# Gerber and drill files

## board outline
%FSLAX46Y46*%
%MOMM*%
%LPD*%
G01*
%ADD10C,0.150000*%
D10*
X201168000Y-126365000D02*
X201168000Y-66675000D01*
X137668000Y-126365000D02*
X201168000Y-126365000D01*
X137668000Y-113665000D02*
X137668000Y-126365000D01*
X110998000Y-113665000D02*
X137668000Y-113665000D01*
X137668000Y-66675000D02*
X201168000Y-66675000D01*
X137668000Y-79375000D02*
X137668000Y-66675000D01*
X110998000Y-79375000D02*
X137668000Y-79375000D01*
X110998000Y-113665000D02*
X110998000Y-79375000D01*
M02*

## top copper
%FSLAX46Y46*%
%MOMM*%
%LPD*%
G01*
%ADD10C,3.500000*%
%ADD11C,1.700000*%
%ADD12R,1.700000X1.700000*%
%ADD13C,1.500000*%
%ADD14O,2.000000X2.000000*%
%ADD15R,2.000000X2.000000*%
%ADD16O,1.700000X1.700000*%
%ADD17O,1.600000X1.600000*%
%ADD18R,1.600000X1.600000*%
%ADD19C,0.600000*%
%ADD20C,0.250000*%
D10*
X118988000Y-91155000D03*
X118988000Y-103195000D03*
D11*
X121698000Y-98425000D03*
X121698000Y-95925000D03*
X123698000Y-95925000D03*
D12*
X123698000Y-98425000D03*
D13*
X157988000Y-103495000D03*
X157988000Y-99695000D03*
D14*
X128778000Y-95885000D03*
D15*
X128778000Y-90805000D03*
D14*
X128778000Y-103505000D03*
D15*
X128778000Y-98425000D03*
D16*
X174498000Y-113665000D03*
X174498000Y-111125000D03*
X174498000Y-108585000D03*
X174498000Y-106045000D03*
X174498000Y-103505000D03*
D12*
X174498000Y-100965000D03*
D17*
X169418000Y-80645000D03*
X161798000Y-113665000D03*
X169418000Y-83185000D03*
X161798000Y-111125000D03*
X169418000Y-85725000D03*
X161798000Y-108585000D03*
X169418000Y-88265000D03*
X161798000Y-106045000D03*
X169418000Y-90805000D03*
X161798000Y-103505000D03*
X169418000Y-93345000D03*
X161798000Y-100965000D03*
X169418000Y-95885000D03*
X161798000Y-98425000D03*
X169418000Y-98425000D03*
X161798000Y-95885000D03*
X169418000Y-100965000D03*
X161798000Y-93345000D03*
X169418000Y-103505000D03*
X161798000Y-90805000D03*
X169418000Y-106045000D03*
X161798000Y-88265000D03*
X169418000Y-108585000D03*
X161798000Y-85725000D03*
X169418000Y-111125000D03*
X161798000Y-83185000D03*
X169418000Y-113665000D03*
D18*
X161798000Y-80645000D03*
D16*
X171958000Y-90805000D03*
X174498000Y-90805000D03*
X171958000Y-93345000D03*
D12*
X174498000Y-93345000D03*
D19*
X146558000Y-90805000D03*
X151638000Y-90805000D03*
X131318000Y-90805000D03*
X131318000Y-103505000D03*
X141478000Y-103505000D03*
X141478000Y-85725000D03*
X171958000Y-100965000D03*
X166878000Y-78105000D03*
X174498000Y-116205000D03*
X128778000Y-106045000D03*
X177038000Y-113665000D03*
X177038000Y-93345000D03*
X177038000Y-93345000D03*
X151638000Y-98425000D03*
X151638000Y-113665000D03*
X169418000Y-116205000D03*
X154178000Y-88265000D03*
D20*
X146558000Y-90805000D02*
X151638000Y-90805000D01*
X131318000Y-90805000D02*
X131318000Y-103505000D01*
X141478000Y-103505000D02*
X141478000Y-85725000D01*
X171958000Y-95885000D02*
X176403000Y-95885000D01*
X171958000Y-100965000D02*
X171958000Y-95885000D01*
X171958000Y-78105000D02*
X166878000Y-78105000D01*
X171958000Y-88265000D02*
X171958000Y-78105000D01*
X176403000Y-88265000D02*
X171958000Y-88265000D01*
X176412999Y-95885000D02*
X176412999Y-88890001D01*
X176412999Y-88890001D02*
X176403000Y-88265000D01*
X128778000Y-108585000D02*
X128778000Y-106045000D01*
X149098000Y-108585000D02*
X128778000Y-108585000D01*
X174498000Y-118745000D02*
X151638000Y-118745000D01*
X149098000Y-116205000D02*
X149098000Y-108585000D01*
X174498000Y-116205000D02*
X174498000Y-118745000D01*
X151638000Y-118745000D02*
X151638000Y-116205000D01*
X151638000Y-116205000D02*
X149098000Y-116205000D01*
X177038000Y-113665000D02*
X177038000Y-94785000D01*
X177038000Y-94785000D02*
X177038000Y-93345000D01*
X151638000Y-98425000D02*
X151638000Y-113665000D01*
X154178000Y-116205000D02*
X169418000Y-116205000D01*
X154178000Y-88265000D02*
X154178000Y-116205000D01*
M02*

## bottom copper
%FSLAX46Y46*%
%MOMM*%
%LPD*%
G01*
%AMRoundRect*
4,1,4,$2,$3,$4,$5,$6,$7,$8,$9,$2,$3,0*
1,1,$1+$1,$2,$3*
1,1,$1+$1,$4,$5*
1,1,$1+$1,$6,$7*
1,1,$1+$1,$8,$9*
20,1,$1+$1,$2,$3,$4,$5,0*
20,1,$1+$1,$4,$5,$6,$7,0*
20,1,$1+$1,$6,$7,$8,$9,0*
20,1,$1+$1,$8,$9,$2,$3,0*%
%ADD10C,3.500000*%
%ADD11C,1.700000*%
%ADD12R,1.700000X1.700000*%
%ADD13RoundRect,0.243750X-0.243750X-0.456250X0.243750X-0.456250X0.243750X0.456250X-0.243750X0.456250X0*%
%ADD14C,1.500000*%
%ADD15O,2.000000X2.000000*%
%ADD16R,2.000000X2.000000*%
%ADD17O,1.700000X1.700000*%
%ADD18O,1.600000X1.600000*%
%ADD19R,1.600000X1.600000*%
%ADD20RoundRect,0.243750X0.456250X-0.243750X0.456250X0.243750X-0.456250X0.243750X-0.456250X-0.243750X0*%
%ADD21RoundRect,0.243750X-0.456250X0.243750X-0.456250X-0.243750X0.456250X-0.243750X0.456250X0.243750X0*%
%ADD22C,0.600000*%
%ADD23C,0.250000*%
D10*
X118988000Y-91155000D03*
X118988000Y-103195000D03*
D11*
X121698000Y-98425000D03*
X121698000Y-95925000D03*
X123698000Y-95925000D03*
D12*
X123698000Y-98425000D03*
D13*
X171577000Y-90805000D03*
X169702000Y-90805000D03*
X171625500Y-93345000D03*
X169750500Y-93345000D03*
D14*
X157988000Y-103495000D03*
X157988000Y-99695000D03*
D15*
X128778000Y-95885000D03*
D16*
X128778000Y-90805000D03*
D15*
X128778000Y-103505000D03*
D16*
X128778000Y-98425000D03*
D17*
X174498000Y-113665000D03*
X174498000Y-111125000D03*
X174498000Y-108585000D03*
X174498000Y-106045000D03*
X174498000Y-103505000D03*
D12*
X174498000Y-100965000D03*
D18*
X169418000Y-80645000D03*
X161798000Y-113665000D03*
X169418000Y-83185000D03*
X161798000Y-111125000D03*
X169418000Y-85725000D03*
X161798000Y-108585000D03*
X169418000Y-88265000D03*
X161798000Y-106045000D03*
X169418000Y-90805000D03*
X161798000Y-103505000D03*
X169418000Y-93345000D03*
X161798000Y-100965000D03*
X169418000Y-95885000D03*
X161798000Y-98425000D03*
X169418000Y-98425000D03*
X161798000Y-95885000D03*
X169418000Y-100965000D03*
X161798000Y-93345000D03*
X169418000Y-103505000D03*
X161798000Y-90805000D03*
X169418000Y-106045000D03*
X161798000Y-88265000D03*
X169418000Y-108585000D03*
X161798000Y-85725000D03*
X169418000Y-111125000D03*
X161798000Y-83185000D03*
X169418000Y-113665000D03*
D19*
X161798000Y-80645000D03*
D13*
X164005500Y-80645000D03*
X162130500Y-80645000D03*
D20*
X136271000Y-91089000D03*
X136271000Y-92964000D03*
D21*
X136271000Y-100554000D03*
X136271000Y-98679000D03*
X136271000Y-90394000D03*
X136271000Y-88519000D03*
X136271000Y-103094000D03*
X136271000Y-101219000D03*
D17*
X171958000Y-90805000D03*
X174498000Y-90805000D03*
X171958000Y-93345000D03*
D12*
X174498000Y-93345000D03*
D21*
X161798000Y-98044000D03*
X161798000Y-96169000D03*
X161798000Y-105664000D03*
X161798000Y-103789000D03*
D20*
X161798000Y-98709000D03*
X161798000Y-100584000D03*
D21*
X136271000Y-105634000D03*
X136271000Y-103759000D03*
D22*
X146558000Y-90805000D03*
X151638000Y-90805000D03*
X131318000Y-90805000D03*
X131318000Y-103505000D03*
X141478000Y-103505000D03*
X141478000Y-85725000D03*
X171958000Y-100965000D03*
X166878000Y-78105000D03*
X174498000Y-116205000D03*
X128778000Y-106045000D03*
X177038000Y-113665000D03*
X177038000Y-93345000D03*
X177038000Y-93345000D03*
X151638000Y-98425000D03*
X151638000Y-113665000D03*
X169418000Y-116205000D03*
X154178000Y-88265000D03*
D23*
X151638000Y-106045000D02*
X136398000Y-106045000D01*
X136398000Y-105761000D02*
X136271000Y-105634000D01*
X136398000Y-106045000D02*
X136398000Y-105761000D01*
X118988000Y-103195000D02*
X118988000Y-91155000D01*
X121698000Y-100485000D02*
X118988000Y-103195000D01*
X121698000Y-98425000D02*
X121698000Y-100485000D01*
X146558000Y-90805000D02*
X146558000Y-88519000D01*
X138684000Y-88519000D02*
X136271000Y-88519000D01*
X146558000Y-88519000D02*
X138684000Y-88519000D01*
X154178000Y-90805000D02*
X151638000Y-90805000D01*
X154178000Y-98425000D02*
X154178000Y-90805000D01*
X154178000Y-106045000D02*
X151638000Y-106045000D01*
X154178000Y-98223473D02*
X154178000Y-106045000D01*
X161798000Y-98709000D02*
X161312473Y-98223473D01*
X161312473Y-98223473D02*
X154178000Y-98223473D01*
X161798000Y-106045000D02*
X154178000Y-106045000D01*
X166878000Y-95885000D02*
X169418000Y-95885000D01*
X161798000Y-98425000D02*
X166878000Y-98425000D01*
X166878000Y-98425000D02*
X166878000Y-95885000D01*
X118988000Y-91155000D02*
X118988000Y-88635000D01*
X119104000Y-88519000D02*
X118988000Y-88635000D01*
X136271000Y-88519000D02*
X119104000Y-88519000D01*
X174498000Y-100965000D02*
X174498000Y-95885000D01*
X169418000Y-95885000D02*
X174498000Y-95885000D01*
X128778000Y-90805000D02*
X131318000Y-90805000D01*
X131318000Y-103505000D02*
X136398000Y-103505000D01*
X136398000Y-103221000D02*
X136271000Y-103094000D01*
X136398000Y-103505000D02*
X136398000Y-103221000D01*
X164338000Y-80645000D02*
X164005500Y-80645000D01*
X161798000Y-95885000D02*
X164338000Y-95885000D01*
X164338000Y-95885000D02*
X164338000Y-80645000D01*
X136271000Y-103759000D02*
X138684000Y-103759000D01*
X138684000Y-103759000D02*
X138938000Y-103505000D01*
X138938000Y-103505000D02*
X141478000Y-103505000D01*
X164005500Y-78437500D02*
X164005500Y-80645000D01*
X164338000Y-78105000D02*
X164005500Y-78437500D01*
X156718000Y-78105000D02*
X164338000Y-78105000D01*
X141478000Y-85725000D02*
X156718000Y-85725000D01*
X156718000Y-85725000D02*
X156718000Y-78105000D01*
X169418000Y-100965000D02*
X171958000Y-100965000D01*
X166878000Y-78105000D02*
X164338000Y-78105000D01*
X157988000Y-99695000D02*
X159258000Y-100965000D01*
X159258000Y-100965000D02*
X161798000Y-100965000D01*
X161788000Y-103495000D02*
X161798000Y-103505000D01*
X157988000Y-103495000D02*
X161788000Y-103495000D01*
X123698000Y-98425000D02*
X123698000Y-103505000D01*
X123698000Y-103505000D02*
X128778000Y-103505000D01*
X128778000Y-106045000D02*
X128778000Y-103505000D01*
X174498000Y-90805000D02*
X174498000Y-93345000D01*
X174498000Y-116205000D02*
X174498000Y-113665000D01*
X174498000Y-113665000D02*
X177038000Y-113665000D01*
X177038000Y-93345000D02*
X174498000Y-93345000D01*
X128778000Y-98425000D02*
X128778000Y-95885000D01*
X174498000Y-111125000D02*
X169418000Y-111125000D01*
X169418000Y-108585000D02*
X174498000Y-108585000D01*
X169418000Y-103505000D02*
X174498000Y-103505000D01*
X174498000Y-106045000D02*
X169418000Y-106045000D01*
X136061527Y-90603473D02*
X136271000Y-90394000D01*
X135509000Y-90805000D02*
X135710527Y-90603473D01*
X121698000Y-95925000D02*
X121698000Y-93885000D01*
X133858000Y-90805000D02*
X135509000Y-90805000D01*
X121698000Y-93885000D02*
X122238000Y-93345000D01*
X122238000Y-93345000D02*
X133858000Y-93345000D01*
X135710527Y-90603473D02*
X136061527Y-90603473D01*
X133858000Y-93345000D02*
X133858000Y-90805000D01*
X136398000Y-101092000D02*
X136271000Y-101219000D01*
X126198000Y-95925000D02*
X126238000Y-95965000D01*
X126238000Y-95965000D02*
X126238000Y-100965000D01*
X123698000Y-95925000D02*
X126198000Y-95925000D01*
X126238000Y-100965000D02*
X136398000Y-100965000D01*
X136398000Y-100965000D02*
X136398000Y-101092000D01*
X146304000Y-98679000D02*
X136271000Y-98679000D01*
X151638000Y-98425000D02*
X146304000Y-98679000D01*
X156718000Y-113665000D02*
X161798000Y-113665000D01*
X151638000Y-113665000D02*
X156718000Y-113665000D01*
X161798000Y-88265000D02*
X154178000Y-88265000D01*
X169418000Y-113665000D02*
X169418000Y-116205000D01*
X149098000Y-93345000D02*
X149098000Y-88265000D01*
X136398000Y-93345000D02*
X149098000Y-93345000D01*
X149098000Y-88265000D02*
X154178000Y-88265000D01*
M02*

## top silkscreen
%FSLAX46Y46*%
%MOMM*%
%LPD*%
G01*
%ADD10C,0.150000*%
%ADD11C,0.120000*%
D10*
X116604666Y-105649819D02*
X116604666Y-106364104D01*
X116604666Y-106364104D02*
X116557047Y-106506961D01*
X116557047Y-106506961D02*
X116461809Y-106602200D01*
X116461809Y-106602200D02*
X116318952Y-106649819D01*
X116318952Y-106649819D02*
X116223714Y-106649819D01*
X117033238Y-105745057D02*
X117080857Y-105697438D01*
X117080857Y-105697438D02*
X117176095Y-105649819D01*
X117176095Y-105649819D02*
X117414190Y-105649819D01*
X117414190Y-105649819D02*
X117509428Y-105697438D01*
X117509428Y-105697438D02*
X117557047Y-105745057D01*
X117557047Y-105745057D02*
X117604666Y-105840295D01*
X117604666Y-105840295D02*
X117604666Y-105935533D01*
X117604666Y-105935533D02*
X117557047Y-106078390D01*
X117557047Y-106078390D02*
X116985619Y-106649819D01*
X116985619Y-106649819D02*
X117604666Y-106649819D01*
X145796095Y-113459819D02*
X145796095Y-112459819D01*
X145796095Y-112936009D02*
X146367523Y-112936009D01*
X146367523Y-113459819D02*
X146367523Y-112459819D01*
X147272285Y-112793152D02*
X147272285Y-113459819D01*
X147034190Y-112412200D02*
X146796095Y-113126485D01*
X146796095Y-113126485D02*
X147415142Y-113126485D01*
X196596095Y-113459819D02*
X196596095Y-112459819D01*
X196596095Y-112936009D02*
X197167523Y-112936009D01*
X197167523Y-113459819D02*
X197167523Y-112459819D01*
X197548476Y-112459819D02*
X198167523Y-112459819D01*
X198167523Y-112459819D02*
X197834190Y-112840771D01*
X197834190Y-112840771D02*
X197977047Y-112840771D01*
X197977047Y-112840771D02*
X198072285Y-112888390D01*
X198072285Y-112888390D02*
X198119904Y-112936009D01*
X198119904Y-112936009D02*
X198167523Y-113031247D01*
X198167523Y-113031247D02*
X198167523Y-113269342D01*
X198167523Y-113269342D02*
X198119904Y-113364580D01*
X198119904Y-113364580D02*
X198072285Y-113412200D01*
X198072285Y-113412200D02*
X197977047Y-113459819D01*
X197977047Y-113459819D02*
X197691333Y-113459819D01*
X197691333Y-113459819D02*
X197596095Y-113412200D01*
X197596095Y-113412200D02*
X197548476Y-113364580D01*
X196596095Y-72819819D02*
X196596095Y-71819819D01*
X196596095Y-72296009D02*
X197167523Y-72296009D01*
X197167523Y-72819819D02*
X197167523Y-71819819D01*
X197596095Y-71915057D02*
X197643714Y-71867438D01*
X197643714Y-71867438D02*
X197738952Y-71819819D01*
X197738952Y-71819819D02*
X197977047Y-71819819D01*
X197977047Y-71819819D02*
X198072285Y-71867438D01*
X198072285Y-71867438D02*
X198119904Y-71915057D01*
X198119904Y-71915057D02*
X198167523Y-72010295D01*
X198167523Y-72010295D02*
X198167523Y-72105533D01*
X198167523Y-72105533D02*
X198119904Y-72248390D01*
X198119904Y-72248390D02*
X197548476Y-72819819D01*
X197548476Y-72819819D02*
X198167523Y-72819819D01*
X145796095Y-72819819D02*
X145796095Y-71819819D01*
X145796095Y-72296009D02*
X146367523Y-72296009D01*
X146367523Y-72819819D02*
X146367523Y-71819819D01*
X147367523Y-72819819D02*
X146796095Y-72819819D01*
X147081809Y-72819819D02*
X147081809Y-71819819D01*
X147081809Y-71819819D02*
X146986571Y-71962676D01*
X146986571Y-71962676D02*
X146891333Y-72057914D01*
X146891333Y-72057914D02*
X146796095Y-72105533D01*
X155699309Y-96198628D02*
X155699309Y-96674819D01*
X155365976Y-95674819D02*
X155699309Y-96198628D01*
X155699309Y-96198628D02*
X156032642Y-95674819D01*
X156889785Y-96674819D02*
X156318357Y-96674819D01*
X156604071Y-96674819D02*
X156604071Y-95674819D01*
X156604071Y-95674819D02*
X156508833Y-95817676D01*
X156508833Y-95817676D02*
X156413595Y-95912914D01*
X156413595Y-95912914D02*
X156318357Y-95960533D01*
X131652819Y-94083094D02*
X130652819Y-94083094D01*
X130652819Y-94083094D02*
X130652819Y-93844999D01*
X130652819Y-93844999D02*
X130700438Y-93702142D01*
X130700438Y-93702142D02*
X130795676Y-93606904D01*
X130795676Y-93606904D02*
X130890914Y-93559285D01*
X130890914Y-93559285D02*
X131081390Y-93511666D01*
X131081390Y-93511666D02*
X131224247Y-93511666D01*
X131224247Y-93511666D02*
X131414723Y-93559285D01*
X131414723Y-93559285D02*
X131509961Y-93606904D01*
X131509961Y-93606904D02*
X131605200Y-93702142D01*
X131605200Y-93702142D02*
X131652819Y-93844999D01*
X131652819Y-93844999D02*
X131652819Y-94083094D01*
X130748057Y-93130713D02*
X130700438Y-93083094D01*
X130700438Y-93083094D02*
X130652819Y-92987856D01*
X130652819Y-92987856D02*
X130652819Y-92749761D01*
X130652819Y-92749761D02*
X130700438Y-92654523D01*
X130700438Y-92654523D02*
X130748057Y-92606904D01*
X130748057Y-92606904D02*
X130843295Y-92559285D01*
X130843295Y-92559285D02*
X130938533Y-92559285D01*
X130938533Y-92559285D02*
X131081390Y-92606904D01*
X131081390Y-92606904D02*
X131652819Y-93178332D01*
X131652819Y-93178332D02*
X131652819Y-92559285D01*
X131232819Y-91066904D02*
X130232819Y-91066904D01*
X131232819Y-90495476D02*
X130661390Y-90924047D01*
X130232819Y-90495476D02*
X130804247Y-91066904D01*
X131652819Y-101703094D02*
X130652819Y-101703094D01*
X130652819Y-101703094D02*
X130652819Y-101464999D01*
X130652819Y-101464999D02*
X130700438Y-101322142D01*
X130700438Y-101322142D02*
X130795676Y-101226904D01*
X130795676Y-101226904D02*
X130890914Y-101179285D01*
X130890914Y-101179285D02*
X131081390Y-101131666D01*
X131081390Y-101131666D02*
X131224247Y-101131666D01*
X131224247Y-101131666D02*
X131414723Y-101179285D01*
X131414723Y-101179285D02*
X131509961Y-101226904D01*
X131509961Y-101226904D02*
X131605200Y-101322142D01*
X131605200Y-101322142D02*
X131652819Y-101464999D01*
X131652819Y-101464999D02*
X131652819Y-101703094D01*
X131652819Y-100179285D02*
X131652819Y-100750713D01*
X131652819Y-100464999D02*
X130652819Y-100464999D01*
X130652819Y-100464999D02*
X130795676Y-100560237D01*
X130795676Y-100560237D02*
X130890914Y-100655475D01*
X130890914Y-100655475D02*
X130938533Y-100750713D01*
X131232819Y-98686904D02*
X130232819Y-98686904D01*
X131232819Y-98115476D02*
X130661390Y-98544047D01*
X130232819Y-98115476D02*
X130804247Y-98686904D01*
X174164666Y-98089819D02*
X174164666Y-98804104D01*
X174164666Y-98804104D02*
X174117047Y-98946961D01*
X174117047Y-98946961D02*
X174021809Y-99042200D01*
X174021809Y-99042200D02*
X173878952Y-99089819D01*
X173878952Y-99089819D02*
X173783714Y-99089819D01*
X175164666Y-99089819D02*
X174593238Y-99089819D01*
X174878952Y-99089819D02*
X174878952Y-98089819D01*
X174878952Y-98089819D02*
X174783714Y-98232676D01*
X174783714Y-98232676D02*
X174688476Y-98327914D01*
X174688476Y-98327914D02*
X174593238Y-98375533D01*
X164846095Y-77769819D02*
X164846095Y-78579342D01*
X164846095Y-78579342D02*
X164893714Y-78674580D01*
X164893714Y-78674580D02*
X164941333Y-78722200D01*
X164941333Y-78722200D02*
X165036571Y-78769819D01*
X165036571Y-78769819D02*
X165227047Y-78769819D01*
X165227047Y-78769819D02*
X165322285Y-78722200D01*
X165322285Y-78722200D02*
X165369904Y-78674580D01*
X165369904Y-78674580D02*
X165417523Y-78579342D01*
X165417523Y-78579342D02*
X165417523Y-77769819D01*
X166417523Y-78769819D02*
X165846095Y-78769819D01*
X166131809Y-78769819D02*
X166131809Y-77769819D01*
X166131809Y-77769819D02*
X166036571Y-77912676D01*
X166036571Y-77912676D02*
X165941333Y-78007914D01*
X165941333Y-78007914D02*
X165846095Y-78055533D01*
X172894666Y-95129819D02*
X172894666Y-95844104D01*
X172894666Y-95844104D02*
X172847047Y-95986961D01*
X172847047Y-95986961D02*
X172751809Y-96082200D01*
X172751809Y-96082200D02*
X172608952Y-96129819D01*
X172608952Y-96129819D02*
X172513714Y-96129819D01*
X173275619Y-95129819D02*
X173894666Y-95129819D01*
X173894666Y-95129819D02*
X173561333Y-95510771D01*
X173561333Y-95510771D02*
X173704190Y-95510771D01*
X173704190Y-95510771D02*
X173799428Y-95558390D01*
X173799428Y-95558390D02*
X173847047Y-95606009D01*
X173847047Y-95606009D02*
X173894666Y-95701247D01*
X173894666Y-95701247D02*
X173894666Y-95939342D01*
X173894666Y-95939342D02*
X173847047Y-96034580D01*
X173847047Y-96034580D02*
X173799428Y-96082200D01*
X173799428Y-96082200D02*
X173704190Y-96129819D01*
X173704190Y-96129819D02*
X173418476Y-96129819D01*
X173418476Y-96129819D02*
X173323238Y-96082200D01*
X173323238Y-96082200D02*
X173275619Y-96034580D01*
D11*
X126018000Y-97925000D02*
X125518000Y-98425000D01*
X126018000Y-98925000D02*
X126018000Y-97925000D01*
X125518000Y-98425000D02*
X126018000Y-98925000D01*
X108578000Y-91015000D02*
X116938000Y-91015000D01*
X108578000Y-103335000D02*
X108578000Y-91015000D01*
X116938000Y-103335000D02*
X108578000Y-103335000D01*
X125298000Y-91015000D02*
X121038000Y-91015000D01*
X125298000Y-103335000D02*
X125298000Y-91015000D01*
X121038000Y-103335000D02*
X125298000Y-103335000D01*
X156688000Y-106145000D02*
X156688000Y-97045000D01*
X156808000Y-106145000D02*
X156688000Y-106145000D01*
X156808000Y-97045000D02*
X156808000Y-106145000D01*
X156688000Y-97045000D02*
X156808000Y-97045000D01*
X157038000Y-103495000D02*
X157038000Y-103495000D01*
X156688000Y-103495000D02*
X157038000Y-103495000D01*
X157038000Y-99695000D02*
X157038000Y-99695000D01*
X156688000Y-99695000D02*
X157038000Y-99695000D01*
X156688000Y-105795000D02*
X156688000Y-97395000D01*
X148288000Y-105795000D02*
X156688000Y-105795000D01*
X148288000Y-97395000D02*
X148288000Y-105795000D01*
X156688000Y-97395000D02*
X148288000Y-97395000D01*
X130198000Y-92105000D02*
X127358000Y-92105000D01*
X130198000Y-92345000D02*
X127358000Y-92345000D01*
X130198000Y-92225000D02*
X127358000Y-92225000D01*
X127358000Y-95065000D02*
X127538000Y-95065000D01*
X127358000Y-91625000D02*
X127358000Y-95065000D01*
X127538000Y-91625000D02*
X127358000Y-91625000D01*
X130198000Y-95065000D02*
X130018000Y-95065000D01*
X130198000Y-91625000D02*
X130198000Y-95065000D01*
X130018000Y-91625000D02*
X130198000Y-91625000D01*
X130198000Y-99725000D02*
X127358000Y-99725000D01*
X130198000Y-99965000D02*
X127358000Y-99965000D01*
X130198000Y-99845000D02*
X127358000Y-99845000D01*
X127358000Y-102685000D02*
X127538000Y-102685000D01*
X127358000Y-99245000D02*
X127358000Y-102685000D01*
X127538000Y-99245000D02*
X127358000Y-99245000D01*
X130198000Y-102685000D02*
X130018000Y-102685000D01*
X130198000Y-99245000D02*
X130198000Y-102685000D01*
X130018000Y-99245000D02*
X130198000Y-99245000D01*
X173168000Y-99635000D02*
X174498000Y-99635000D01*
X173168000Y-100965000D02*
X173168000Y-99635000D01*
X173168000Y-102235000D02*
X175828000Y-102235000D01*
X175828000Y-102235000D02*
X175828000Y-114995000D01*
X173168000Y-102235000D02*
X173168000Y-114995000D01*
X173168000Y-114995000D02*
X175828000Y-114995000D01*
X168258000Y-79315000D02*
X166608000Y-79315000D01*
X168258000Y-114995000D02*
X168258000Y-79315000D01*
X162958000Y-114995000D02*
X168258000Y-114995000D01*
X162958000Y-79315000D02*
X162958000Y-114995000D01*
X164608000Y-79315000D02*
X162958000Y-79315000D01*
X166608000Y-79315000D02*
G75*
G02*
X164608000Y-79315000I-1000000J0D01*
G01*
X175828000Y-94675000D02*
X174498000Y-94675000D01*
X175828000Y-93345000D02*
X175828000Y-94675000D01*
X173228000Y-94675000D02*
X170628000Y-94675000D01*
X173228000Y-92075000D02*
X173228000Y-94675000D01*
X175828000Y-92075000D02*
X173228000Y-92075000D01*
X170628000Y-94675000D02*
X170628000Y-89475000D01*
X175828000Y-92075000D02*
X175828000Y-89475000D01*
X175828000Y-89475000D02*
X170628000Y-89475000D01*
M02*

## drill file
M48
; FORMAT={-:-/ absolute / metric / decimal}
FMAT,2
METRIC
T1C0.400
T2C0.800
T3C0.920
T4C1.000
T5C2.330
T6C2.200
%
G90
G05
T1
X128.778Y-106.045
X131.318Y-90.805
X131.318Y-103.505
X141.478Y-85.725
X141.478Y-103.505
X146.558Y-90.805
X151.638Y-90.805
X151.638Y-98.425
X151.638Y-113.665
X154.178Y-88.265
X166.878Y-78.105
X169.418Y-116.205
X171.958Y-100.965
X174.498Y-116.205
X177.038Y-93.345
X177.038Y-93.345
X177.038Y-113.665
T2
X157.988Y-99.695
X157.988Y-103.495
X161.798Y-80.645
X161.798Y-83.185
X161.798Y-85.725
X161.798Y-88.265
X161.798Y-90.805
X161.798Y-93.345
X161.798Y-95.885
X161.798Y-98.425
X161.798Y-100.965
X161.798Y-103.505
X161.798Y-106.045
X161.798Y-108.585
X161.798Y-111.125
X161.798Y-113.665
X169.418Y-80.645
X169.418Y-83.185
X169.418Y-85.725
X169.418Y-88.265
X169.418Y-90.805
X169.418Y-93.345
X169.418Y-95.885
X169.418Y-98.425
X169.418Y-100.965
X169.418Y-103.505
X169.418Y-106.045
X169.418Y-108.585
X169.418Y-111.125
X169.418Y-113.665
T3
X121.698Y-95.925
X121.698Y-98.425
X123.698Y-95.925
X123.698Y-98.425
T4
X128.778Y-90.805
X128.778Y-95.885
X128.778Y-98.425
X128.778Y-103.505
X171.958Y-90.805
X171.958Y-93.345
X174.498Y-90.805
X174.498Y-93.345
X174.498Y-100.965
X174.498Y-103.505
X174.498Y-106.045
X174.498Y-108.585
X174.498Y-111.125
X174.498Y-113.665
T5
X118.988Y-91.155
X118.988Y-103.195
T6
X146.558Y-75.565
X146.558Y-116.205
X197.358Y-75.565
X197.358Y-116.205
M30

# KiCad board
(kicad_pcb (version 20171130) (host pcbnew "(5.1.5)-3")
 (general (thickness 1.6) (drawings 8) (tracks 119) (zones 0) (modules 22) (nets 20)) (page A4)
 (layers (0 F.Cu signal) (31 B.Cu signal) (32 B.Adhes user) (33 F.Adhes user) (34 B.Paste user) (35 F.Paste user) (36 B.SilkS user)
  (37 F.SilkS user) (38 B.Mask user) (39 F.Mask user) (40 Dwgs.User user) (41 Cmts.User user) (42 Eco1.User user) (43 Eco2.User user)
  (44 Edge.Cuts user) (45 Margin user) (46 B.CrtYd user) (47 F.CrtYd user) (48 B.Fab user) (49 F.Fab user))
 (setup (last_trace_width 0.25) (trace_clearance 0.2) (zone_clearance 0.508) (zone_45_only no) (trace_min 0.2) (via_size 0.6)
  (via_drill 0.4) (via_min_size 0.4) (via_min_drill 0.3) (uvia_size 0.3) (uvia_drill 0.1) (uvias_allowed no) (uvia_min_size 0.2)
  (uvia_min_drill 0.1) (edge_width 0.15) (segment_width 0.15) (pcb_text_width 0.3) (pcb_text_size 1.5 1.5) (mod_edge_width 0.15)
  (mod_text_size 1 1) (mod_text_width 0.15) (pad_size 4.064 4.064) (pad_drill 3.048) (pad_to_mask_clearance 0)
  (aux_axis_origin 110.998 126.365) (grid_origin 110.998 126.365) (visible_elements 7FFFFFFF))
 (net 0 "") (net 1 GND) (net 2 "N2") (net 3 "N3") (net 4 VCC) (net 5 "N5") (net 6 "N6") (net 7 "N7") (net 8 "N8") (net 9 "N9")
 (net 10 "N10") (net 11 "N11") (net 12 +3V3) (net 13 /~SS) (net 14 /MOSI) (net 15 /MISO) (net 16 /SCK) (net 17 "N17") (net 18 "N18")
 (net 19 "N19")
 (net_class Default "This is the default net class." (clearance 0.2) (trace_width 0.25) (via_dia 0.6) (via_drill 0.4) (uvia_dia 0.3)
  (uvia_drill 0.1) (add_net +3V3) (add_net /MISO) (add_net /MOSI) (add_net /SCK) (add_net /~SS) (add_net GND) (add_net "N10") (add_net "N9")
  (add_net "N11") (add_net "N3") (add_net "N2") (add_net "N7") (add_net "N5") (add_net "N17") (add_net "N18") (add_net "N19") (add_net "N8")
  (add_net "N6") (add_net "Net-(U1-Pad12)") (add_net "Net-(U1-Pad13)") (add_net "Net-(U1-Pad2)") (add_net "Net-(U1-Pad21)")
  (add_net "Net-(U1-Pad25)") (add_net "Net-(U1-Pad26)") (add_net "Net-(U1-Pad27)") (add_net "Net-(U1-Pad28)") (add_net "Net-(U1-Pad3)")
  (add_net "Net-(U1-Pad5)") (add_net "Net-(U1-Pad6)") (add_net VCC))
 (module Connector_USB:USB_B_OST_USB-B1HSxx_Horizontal (layer F.Cu) (at 123.698 98.425 180)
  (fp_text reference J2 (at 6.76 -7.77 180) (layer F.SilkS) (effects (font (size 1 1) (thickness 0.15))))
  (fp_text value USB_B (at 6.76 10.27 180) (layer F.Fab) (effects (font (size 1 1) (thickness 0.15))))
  (fp_line (start -2.32 0.5) (end -1.82 0) (layer F.SilkS) (width 0.12))
  (fp_line (start -2.32 -0.5) (end -2.32 0.5) (layer F.SilkS) (width 0.12))
  (fp_line (start -1.82 0) (end -2.32 -0.5) (layer F.SilkS) (width 0.12))
  (fp_line (start 15.12 7.41) (end 6.76 7.41) (layer F.SilkS) (width 0.12))
  (fp_line (start 15.12 -4.91) (end 15.12 7.41) (layer F.SilkS) (width 0.12))
  (fp_line (start 6.76 -4.91) (end 15.12 -4.91) (layer F.SilkS) (width 0.12))
  (fp_line (start -1.6 7.41) (end 2.66 7.41) (layer F.SilkS) (width 0.12))
  (fp_line (start -1.6 -4.91) (end -1.6 7.41) (layer F.SilkS) (width 0.12))
  (fp_line (start 2.66 -4.91) (end -1.6 -4.91) (layer F.SilkS) (width 0.12))
  (pad 5 thru_hole circle (at 4.71 7.27 180) (size 3.5 3.5) (drill 2.33) (layers *.Cu *.Mask) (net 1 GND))
  (pad 5 thru_hole circle (at 4.71 -4.77 180) (size 3.5 3.5) (drill 2.33) (layers *.Cu *.Mask) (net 1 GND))
  (pad 4 thru_hole circle (at 2 0 180) (size 1.7 1.7) (drill 0.92) (layers *.Cu *.Mask) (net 1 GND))
  (pad 3 thru_hole circle (at 2 2.5 180) (size 1.7 1.7) (drill 0.92) (layers *.Cu *.Mask) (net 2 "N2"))
  (pad 2 thru_hole circle (at 0 2.5 180) (size 1.7 1.7) (drill 0.92) (layers *.Cu *.Mask) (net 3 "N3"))
  (pad 1 thru_hole rect (at 0 0 180) (size 1.7 1.7) (drill 0.92) (layers *.Cu *.Mask) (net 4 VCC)))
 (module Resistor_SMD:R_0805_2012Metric (layer B.Cu) (at 170.6395 90.805)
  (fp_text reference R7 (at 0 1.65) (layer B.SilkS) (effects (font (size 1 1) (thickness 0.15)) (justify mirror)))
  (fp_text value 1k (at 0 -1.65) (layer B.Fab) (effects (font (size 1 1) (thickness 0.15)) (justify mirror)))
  (pad 2 smd roundrect (at 0.9375 0) (size 0.975 1.4) (layers B.Cu B.Paste B.Mask) (roundrect_rratio 0.25) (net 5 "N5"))
  (pad 1 smd roundrect (at -0.9375 0) (size 0.975 1.4) (layers B.Cu B.Paste B.Mask) (roundrect_rratio 0.25) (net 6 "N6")))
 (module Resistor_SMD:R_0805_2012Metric (layer B.Cu) (at 170.688 93.345)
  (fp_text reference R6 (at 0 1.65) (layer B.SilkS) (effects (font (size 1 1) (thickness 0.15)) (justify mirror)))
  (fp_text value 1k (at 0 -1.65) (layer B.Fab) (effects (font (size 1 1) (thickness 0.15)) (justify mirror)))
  (pad 2 smd roundrect (at 0.9375 0) (size 0.975 1.4) (layers B.Cu B.Paste B.Mask) (roundrect_rratio 0.25) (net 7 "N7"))
  (pad 1 smd roundrect (at -0.9375 0) (size 0.975 1.4) (layers B.Cu B.Paste B.Mask) (roundrect_rratio 0.25) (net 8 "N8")))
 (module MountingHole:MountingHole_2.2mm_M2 (layer F.Cu) (at 146.558 116.205)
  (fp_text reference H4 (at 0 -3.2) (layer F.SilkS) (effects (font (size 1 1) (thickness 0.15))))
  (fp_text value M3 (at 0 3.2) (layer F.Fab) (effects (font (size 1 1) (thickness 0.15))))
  (pad 1 np_thru_hole circle (at 0 0) (size 2.2 2.2) (drill 2.2) (layers *.Cu *.Mask)))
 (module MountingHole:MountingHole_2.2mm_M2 (layer F.Cu) (at 197.358 116.205)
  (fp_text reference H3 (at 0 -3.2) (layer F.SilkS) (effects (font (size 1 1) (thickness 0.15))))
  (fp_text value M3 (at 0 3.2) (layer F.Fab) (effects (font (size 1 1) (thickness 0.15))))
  (pad 1 np_thru_hole circle (at 0 0) (size 2.2 2.2) (drill 2.2) (layers *.Cu *.Mask)))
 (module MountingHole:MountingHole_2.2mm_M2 (layer F.Cu) (at 197.358 75.565)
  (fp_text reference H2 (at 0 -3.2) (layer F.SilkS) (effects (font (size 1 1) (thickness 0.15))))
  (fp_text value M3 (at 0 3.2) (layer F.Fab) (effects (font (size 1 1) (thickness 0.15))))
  (pad 1 np_thru_hole circle (at 0 0) (size 2.2 2.2) (drill 2.2) (layers *.Cu *.Mask)))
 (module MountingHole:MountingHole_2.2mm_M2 (layer F.Cu) (at 146.558 75.565)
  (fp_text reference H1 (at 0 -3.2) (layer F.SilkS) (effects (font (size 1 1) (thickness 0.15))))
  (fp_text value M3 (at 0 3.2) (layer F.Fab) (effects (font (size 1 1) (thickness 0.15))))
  (pad 1 np_thru_hole circle (at 0 0) (size 2.2 2.2) (drill 2.2) (layers *.Cu *.Mask)))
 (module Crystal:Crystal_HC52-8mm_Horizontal (layer F.Cu) (at 157.988 99.695 270)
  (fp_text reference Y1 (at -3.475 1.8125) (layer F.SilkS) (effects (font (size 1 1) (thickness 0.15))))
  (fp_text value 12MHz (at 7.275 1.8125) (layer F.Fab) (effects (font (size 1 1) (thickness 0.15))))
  (fp_line (start 6.45 1.3) (end -2.65 1.3) (layer F.SilkS) (width 0.12))
  (fp_line (start 6.45 1.18) (end 6.45 1.3) (layer F.SilkS) (width 0.12))
  (fp_line (start -2.65 1.18) (end 6.45 1.18) (layer F.SilkS) (width 0.12))
  (fp_line (start -2.65 1.3) (end -2.65 1.18) (layer F.SilkS) (width 0.12))
  (fp_line (start 3.8 0.95) (end 3.8 0.95) (layer F.SilkS) (width 0.12))
  (fp_line (start 3.8 1.3) (end 3.8 0.95) (layer F.SilkS) (width 0.12))
  (fp_line (start 0 0.95) (end 0 0.95) (layer F.SilkS) (width 0.12))
  (fp_line (start 0 1.3) (end 0 0.95) (layer F.SilkS) (width 0.12))
  (fp_line (start 6.1 1.3) (end -2.3 1.3) (layer F.SilkS) (width 0.12))
  (fp_line (start 6.1 9.7) (end 6.1 1.3) (layer F.SilkS) (width 0.12))
  (fp_line (start -2.3 9.7) (end 6.1 9.7) (layer F.SilkS) (width 0.12))
  (fp_line (start -2.3 1.3) (end -2.3 9.7) (layer F.SilkS) (width 0.12))
  (pad 2 thru_hole circle (at 3.8 0 270) (size 1.5 1.5) (drill 0.8) (layers *.Cu *.Mask) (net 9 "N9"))
  (pad 1 thru_hole circle (at 0 0 270) (size 1.5 1.5) (drill 0.8) (layers *.Cu *.Mask) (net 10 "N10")))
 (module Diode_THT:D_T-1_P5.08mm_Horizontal (layer F.Cu) (at 128.778 90.805 270)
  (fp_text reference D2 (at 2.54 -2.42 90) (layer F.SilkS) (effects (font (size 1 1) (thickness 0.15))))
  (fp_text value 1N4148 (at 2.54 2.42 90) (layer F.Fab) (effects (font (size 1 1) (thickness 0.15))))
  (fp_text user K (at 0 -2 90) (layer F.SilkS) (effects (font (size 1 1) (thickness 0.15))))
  (fp_line (start 1.3 -1.42) (end 1.3 1.42) (layer F.SilkS) (width 0.12))
  (fp_line (start 1.54 -1.42) (end 1.54 1.42) (layer F.SilkS) (width 0.12))
  (fp_line (start 1.42 -1.42) (end 1.42 1.42) (layer F.SilkS) (width 0.12))
  (fp_line (start 4.26 1.42) (end 4.26 1.24) (layer F.SilkS) (width 0.12))
  (fp_line (start 0.82 1.42) (end 4.26 1.42) (layer F.SilkS) (width 0.12))
  (fp_line (start 0.82 1.24) (end 0.82 1.42) (layer F.SilkS) (width 0.12))
  (fp_line (start 4.26 -1.42) (end 4.26 -1.24) (layer F.SilkS) (width 0.12))
  (fp_line (start 0.82 -1.42) (end 4.26 -1.42) (layer F.SilkS) (width 0.12))
  (fp_line (start 0.82 -1.24) (end 0.82 -1.42) (layer F.SilkS) (width 0.12))
  (pad 2 thru_hole oval (at 5.08 0 270) (size 2 2) (drill 1) (layers *.Cu *.Mask) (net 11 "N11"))
  (pad 1 thru_hole rect (at 0 0 270) (size 2 2) (drill 1) (layers *.Cu *.Mask) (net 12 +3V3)))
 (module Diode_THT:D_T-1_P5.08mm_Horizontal (layer F.Cu) (at 128.778 98.425 270)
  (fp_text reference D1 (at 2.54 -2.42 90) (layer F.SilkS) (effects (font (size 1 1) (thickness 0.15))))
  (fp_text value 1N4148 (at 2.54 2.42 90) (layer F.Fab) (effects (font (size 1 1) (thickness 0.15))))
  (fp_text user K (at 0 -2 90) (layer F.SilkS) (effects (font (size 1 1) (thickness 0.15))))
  (fp_line (start 1.3 -1.42) (end 1.3 1.42) (layer F.SilkS) (width 0.12))
  (fp_line (start 1.54 -1.42) (end 1.54 1.42) (layer F.SilkS) (width 0.12))
  (fp_line (start 1.42 -1.42) (end 1.42 1.42) (layer F.SilkS) (width 0.12))
  (fp_line (start 4.26 1.42) (end 4.26 1.24) (layer F.SilkS) (width 0.12))
  (fp_line (start 0.82 1.42) (end 4.26 1.42) (layer F.SilkS) (width 0.12))
  (fp_line (start 0.82 1.24) (end 0.82 1.42) (layer F.SilkS) (width 0.12))
  (fp_line (start 4.26 -1.42) (end 4.26 -1.24) (layer F.SilkS) (width 0.12))
  (fp_line (start 0.82 -1.42) (end 4.26 -1.42) (layer F.SilkS) (width 0.12))
  (fp_line (start 0.82 -1.24) (end 0.82 -1.42) (layer F.SilkS) (width 0.12))
  (pad 2 thru_hole oval (at 5.08 0 270) (size 2 2) (drill 1) (layers *.Cu *.Mask) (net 4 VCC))
  (pad 1 thru_hole rect (at 0 0 270) (size 2 2) (drill 1) (layers *.Cu *.Mask) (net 11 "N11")))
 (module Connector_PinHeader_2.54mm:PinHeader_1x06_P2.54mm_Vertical (layer F.Cu) (at 174.498 100.965)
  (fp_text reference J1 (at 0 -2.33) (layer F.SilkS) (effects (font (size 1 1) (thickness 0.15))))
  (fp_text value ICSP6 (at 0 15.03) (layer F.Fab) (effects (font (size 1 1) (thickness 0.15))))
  (fp_line (start -1.33 -1.33) (end 0 -1.33) (layer F.SilkS) (width 0.12))
  (fp_line (start -1.33 0) (end -1.33 -1.33) (layer F.SilkS) (width 0.12))
  (fp_line (start -1.33 1.27) (end 1.33 1.27) (layer F.SilkS) (width 0.12))
  (fp_line (start 1.33 1.27) (end 1.33 14.03) (layer F.SilkS) (width 0.12))
  (fp_line (start -1.33 1.27) (end -1.33 14.03) (layer F.SilkS) (width 0.12))
  (fp_line (start -1.33 14.03) (end 1.33 14.03) (layer F.SilkS) (width 0.12))
  (pad 6 thru_hole oval (at 0 12.7) (size 1.7 1.7) (drill 1) (layers *.Cu *.Mask) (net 4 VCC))
  (pad 5 thru_hole oval (at 0 10.16) (size 1.7 1.7) (drill 1) (layers *.Cu *.Mask) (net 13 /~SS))
  (pad 4 thru_hole oval (at 0 7.62) (size 1.7 1.7) (drill 1) (layers *.Cu *.Mask) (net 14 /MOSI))
  (pad 3 thru_hole oval (at 0 5.08) (size 1.7 1.7) (drill 1) (layers *.Cu *.Mask) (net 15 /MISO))
  (pad 2 thru_hole oval (at 0 2.54) (size 1.7 1.7) (drill 1) (layers *.Cu *.Mask) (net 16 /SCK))
  (pad 1 thru_hole rect (at 0 0) (size 1.7 1.7) (drill 1) (layers *.Cu *.Mask) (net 1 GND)))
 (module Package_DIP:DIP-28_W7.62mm (layer F.Cu) (at 161.798 80.645)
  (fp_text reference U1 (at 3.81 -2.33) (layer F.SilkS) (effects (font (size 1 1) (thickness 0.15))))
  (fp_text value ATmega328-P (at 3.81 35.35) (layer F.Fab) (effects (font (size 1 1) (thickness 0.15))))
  (fp_line (start 6.46 -1.33) (end 4.81 -1.33) (layer F.SilkS) (width 0.12))
  (fp_line (start 6.46 34.35) (end 6.46 -1.33) (layer F.SilkS) (width 0.12))
  (fp_line (start 1.16 34.35) (end 6.46 34.35) (layer F.SilkS) (width 0.12))
  (fp_line (start 1.16 -1.33) (end 1.16 34.35) (layer F.SilkS) (width 0.12))
  (fp_line (start 2.81 -1.33) (end 1.16 -1.33) (layer F.SilkS) (width 0.12))
  (fp_arc (start 3.81 -1.33) (end 2.81 -1.33) (angle -180) (layer F.SilkS) (width 0.12))
  (pad 28 thru_hole oval (at 7.62 0) (size 1.6 1.6) (drill 0.8) (layers *.Cu *.Mask))
  (pad 14 thru_hole oval (at 0 33.02) (size 1.6 1.6) (drill 0.8) (layers *.Cu *.Mask) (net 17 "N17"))
  (pad 27 thru_hole oval (at 7.62 2.54) (size 1.6 1.6) (drill 0.8) (layers *.Cu *.Mask))
  (pad 13 thru_hole oval (at 0 30.48) (size 1.6 1.6) (drill 0.8) (layers *.Cu *.Mask))
  (pad 26 thru_hole oval (at 7.62 5.08) (size 1.6 1.6) (drill 0.8) (layers *.Cu *.Mask))
  (pad 12 thru_hole oval (at 0 27.94) (size 1.6 1.6) (drill 0.8) (layers *.Cu *.Mask))
  (pad 25 thru_hole oval (at 7.62 7.62) (size 1.6 1.6) (drill 0.8) (layers *.Cu *.Mask))
  (pad 11 thru_hole oval (at 0 25.4) (size 1.6 1.6) (drill 0.8) (layers *.Cu *.Mask) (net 1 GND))
  (pad 24 thru_hole oval (at 7.62 10.16) (size 1.6 1.6) (drill 0.8) (layers *.Cu *.Mask) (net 6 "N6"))
  (pad 10 thru_hole oval (at 0 22.86) (size 1.6 1.6) (drill 0.8) (layers *.Cu *.Mask) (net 9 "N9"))
  (pad 23 thru_hole oval (at 7.62 12.7) (size 1.6 1.6) (drill 0.8) (layers *.Cu *.Mask) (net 8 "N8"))
  (pad 9 thru_hole oval (at 0 20.32) (size 1.6 1.6) (drill 0.8) (layers *.Cu *.Mask) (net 10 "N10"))
  (pad 22 thru_hole oval (at 7.62 15.24) (size 1.6 1.6) (drill 0.8) (layers *.Cu *.Mask) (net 1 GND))
  (pad 8 thru_hole oval (at 0 17.78) (size 1.6 1.6) (drill 0.8) (layers *.Cu *.Mask) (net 1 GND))
  (pad 21 thru_hole oval (at 7.62 17.78) (size 1.6 1.6) (drill 0.8) (layers *.Cu *.Mask))
  (pad 7 thru_hole oval (at 0 15.24) (size 1.6 1.6) (drill 0.8) (layers *.Cu *.Mask) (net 12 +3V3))
  (pad 20 thru_hole oval (at 7.62 20.32) (size 1.6 1.6) (drill 0.8) (layers *.Cu *.Mask) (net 12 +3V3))
  (pad 6 thru_hole oval (at 0 12.7) (size 1.6 1.6) (drill 0.8) (layers *.Cu *.Mask))
  (pad 19 thru_hole oval (at 7.62 22.86) (size 1.6 1.6) (drill 0.8) (layers *.Cu *.Mask) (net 16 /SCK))
  (pad 5 thru_hole oval (at 0 10.16) (size 1.6 1.6) (drill 0.8) (layers *.Cu *.Mask))
  (pad 18 thru_hole oval (at 7.62 25.4) (size 1.6 1.6) (drill 0.8) (layers *.Cu *.Mask) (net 15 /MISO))
  (pad 4 thru_hole oval (at 0 7.62) (size 1.6 1.6) (drill 0.8) (layers *.Cu *.Mask) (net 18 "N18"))
  (pad 17 thru_hole oval (at 7.62 27.94) (size 1.6 1.6) (drill 0.8) (layers *.Cu *.Mask) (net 14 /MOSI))
  (pad 3 thru_hole oval (at 0 5.08) (size 1.6 1.6) (drill 0.8) (layers *.Cu *.Mask))
  (pad 16 thru_hole oval (at 7.62 30.48) (size 1.6 1.6) (drill 0.8) (layers *.Cu *.Mask) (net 13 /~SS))
  (pad 2 thru_hole oval (at 0 2.54) (size 1.6 1.6) (drill 0.8) (layers *.Cu *.Mask))
  (pad 15 thru_hole oval (at 7.62 33.02) (size 1.6 1.6) (drill 0.8) (layers *.Cu *.Mask) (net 18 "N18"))
  (pad 1 thru_hole rect (at 0 0) (size 1.6 1.6) (drill 0.8) (layers *.Cu *.Mask) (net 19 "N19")))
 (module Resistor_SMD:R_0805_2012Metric (layer B.Cu) (at 163.068 80.645)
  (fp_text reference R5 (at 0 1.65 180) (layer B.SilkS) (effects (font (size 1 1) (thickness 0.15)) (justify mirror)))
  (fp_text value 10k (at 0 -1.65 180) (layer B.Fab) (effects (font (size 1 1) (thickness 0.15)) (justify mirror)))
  (pad 2 smd roundrect (at 0.9375 0) (size 0.975 1.4) (layers B.Cu B.Paste B.Mask) (roundrect_rratio 0.25) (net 12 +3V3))
  (pad 1 smd roundrect (at -0.9375 0) (size 0.975 1.4) (layers B.Cu B.Paste B.Mask) (roundrect_rratio 0.25) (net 19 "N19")))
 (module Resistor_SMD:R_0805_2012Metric (layer B.Cu) (at 136.271 92.0265 90)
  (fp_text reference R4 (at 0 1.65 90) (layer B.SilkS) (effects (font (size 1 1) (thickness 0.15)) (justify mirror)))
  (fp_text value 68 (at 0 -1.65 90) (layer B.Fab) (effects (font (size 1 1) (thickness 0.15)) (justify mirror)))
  (pad 2 smd roundrect (at 0.9375 0 90) (size 0.975 1.4) (layers B.Cu B.Paste B.Mask) (roundrect_rratio 0.25) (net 2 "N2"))
  (pad 1 smd roundrect (at -0.9375 0 90) (size 0.975 1.4) (layers B.Cu B.Paste B.Mask) (roundrect_rratio 0.25) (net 18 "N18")))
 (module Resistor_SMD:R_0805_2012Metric (layer B.Cu) (at 136.271 99.6165 270)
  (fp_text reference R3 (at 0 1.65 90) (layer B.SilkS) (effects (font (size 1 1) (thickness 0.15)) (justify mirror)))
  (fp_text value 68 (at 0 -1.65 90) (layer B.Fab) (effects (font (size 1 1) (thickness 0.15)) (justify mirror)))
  (pad 2 smd roundrect (at 0.9375 0 270) (size 0.975 1.4) (layers B.Cu B.Paste B.Mask) (roundrect_rratio 0.25) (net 3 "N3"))
  (pad 1 smd roundrect (at -0.9375 0 270) (size 0.975 1.4) (layers B.Cu B.Paste B.Mask) (roundrect_rratio 0.25) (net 17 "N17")))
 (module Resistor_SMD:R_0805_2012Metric (layer B.Cu) (at 136.271 89.4565 270)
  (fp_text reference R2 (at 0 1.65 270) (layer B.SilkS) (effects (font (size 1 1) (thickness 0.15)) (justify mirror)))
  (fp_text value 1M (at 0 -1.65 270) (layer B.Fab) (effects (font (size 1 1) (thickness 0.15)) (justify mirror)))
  (pad 2 smd roundrect (at 0.9375 0 270) (size 0.975 1.4) (layers B.Cu B.Paste B.Mask) (roundrect_rratio 0.25) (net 2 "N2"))
  (pad 1 smd roundrect (at -0.9375 0 270) (size 0.975 1.4) (layers B.Cu B.Paste B.Mask) (roundrect_rratio 0.25) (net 1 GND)))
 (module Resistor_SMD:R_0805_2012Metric (layer B.Cu) (at 136.271 102.1565 270)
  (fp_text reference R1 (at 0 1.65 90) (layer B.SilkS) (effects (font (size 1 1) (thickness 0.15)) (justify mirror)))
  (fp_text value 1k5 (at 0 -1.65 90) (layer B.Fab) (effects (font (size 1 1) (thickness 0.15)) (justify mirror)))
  (pad 2 smd roundrect (at 0.9375 0 270) (size 0.975 1.4) (layers B.Cu B.Paste B.Mask) (roundrect_rratio 0.25) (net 12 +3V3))
  (pad 1 smd roundrect (at -0.9375 0 270) (size 0.975 1.4) (layers B.Cu B.Paste B.Mask) (roundrect_rratio 0.25) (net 3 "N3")))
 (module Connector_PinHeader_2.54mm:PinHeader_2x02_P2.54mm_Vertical (layer F.Cu) (at 174.498 93.345 180)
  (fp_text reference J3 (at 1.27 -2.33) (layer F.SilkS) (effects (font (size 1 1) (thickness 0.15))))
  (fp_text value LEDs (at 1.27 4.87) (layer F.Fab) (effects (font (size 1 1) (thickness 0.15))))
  (fp_line (start -1.33 -1.33) (end 0 -1.33) (layer F.SilkS) (width 0.12))
  (fp_line (start -1.33 0) (end -1.33 -1.33) (layer F.SilkS) (width 0.12))
  (fp_line (start 1.27 -1.33) (end 3.87 -1.33) (layer F.SilkS) (width 0.12))
  (fp_line (start 1.27 1.27) (end 1.27 -1.33) (layer F.SilkS) (width 0.12))
  (fp_line (start -1.33 1.27) (end 1.27 1.27) (layer F.SilkS) (width 0.12))
  (fp_line (start 3.87 -1.33) (end 3.87 3.87) (layer F.SilkS) (width 0.12))
  (fp_line (start -1.33 1.27) (end -1.33 3.87) (layer F.SilkS) (width 0.12))
  (fp_line (start -1.33 3.87) (end 3.87 3.87) (layer F.SilkS) (width 0.12))
  (pad 4 thru_hole oval (at 2.54 2.54 180) (size 1.7 1.7) (drill 1) (layers *.Cu *.Mask) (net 5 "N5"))
  (pad 3 thru_hole oval (at 0 2.54 180) (size 1.7 1.7) (drill 1) (layers *.Cu *.Mask) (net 4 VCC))
  (pad 2 thru_hole oval (at 2.54 0 180) (size 1.7 1.7) (drill 1) (layers *.Cu *.Mask) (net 7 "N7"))
  (pad 1 thru_hole rect (at 0 0 180) (size 1.7 1.7) (drill 1) (layers *.Cu *.Mask) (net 4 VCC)))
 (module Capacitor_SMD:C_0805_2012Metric (layer B.Cu) (at 161.798 97.1065 270)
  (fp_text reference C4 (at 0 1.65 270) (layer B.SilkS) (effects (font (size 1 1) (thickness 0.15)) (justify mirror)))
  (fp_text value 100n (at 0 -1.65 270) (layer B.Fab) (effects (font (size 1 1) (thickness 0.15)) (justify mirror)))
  (pad 2 smd roundrect (at 0.9375 0 270) (size 0.975 1.4) (layers B.Cu B.Paste B.Mask) (roundrect_rratio 0.25) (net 1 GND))
  (pad 1 smd roundrect (at -0.9375 0 270) (size 0.975 1.4) (layers B.Cu B.Paste B.Mask) (roundrect_rratio 0.25) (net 12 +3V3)))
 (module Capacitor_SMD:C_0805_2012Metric (layer B.Cu) (at 161.798 104.7265 270)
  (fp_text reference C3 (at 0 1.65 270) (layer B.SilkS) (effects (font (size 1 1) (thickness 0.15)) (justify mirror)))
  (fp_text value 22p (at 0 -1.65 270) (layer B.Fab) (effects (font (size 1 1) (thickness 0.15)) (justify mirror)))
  (pad 2 smd roundrect (at 0.9375 0 270) (size 0.975 1.4) (layers B.Cu B.Paste B.Mask) (roundrect_rratio 0.25) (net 1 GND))
  (pad 1 smd roundrect (at -0.9375 0 270) (size 0.975 1.4) (layers B.Cu B.Paste B.Mask) (roundrect_rratio 0.25) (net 9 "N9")))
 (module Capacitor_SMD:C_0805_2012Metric (layer B.Cu) (at 161.798 99.6465 90)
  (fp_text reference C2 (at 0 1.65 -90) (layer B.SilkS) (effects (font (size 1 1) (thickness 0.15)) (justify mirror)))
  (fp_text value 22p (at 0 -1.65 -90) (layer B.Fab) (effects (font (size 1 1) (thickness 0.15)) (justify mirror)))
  (pad 2 smd roundrect (at 0.9375 0 90) (size 0.975 1.4) (layers B.Cu B.Paste B.Mask) (roundrect_rratio 0.25) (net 1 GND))
  (pad 1 smd roundrect (at -0.9375 0 90) (size 0.975 1.4) (layers B.Cu B.Paste B.Mask) (roundrect_rratio 0.25) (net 10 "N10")))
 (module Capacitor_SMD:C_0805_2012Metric (layer B.Cu) (at 136.271 104.6965 270)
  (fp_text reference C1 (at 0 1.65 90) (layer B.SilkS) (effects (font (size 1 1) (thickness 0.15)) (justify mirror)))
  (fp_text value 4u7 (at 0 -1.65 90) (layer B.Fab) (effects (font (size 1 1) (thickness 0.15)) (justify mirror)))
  (pad 2 smd roundrect (at 0.9375 0 270) (size 0.975 1.4) (layers B.Cu B.Paste B.Mask) (roundrect_rratio 0.25) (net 1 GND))
  (pad 1 smd roundrect (at -0.9375 0 270) (size 0.975 1.4) (layers B.Cu B.Paste B.Mask) (roundrect_rratio 0.25) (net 12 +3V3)))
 (gr_line (start 201.168 126.365) (end 201.168 66.675) (layer Edge.Cuts) (width 0.15))
 (gr_line (start 137.668 126.365) (end 201.168 126.365) (layer Edge.Cuts) (width 0.15))
 (gr_line (start 137.668 113.665) (end 137.668 126.365) (layer Edge.Cuts) (width 0.15))
 (gr_line (start 110.998 113.665) (end 137.668 113.665) (layer Edge.Cuts) (width 0.15))
 (gr_line (start 137.668 66.675) (end 201.168 66.675) (layer Edge.Cuts) (width 0.15))
 (gr_line (start 137.668 79.375) (end 137.668 66.675) (layer Edge.Cuts) (width 0.15))
 (gr_line (start 110.998 79.375) (end 137.668 79.375) (layer Edge.Cuts) (width 0.15))
 (gr_line (start 110.998 113.665) (end 110.998 79.375) (layer Edge.Cuts) (width 0.15))
 (segment (start 151.638 106.045) (end 136.398 106.045) (width 0.25) (layer B.Cu) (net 1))
 (segment (start 136.398 105.761) (end 136.271 105.634) (width 0.25) (layer B.Cu) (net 1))
 (segment (start 136.398 106.045) (end 136.398 105.761) (width 0.25) (layer B.Cu) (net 1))
 (segment (start 118.988 103.195) (end 118.988 91.155) (width 0.25) (layer B.Cu) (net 1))
 (segment (start 121.698 100.485) (end 118.988 103.195) (width 0.25) (layer B.Cu) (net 1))
 (segment (start 121.698 98.425) (end 121.698 100.485) (width 0.25) (layer B.Cu) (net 1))
 (via (at 146.558 90.805) (size 0.6) (drill 0.4) (layers F.Cu B.Cu) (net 1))
 (segment (start 146.558 90.805) (end 146.558 88.519) (width 0.25) (layer B.Cu) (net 1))
 (segment (start 138.684 88.519) (end 136.271 88.519) (width 0.25) (layer B.Cu) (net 1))
 (segment (start 146.558 88.519) (end 138.684 88.519) (width 0.25) (layer B.Cu) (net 1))
 (segment (start 146.558 90.805) (end 151.638 90.805) (width 0.25) (layer F.Cu) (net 1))
 (via (at 151.638 90.805) (size 0.6) (drill 0.4) (layers F.Cu B.Cu) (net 1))
 (segment (start 154.178 90.805) (end 151.638 90.805) (width 0.25) (layer B.Cu) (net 1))
 (segment (start 154.178 98.425) (end 154.178 90.805) (width 0.25) (layer B.Cu) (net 1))
 (segment (start 154.178 106.045) (end 151.638 106.045) (width 0.25) (layer B.Cu) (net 1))
 (segment (start 154.178 98.223473) (end 154.178 106.045) (width 0.25) (layer B.Cu) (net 1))
 (segment (start 161.798 98.709) (end 161.312473 98.223473) (width 0.25) (layer B.Cu) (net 1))
 (segment (start 161.312473 98.223473) (end 154.178 98.223473) (width 0.25) (layer B.Cu) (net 1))
 (segment (start 161.798 106.045) (end 154.178 106.045) (width 0.25) (layer B.Cu) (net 1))
 (segment (start 166.878 95.885) (end 169.418 95.885) (width 0.25) (layer B.Cu) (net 1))
 (segment (start 161.798 98.425) (end 166.878 98.425) (width 0.25) (layer B.Cu) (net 1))
 (segment (start 166.878 98.425) (end 166.878 95.885) (width 0.25) (layer B.Cu) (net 1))
 (segment (start 118.988 91.155) (end 118.988 88.635) (width 0.25) (layer B.Cu) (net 1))
 (segment (start 119.104 88.519) (end 118.988 88.635) (width 0.25) (layer B.Cu) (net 1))
 (segment (start 136.271 88.519) (end 119.104 88.519) (width 0.25) (layer B.Cu) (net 1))
 (segment (start 174.498 100.965) (end 174.498 95.885) (width 0.25) (layer B.Cu) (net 1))
 (segment (start 169.418 95.885) (end 174.498 95.885) (width 0.25) (layer B.Cu) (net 1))
 (segment (start 128.778 90.805) (end 131.318 90.805) (width 0.25) (layer B.Cu) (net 12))
 (via (at 131.318 90.805) (size 0.6) (drill 0.4) (layers F.Cu B.Cu) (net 12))
 (segment (start 131.318 90.805) (end 131.318 103.505) (width 0.25) (layer F.Cu) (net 12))
 (via (at 131.318 103.505) (size 0.6) (drill 0.4) (layers F.Cu B.Cu) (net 12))
 (segment (start 131.318 103.505) (end 136.398 103.505) (width 0.25) (layer B.Cu) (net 12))
 (segment (start 136.398 103.221) (end 136.271 103.094) (width 0.25) (layer B.Cu) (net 12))
 (segment (start 136.398 103.505) (end 136.398 103.221) (width 0.25) (layer B.Cu) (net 12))
 (segment (start 164.338 80.645) (end 164.0055 80.645) (width 0.25) (layer B.Cu) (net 12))
 (segment (start 161.798 95.885) (end 164.338 95.885) (width 0.25) (layer B.Cu) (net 12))
 (segment (start 164.338 95.885) (end 164.338 80.645) (width 0.25) (layer B.Cu) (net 12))
 (segment (start 136.271 103.759) (end 138.684 103.759) (width 0.25) (layer B.Cu) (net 12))
 (segment (start 138.684 103.759) (end 138.938 103.505) (width 0.25) (layer B.Cu) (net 12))
 (segment (start 138.938 103.505) (end 141.478 103.505) (width 0.25) (layer B.Cu) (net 12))
 (via (at 141.478 103.505) (size 0.6) (drill 0.4) (layers F.Cu B.Cu) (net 12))
 (segment (start 141.478 103.505) (end 141.478 85.725) (width 0.25) (layer F.Cu) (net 12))
 (via (at 141.478 85.725) (size 0.6) (drill 0.4) (layers F.Cu B.Cu) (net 12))
 (segment (start 164.0055 78.4375) (end 164.0055 80.645) (width 0.25) (layer B.Cu) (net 12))
 (segment (start 164.338 78.105) (end 164.0055 78.4375) (width 0.25) (layer B.Cu) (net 12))
 (segment (start 156.718 78.105) (end 164.338 78.105) (width 0.25) (layer B.Cu) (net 12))
 (segment (start 141.478 85.725) (end 156.718 85.725) (width 0.25) (layer B.Cu) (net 12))
 (segment (start 156.718 85.725) (end 156.718 78.105) (width 0.25) (layer B.Cu) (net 12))
 (segment (start 169.418 100.965) (end 171.958 100.965) (width 0.25) (layer B.Cu) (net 12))
 (via (at 171.958 100.965) (size 0.6) (drill 0.4) (layers F.Cu B.Cu) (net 12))
 (via (at 166.878 78.105) (size 0.6) (drill 0.4) (layers F.Cu B.Cu) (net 12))
 (segment (start 166.878 78.105) (end 164.338 78.105) (width 0.25) (layer B.Cu) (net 12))
 (segment (start 171.958 95.885) (end 176.403 95.885) (width 0.25) (layer F.Cu) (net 12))
 (segment (start 171.958 100.965) (end 171.958 95.885) (width 0.25) (layer F.Cu) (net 12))
 (segment (start 171.958 78.105) (end 166.878 78.105) (width 0.25) (layer F.Cu) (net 12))
 (segment (start 171.958 88.265) (end 171.958 78.105) (width 0.25) (layer F.Cu) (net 12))
 (segment (start 176.403 88.265) (end 171.958 88.265) (width 0.25) (layer F.Cu) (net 12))
 (segment (start 176.412999 95.885) (end 176.412999 88.890001) (width 0.25) (layer F.Cu) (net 12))
 (segment (start 176.412999 88.890001) (end 176.403 88.265) (width 0.25) (layer F.Cu) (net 12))
 (segment (start 157.988 99.695) (end 159.258 100.965) (width 0.25) (layer B.Cu) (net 10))
 (segment (start 159.258 100.965) (end 161.798 100.965) (width 0.25) (layer B.Cu) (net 10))
 (segment (start 161.788 103.495) (end 161.798 103.505) (width 0.25) (layer B.Cu) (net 9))
 (segment (start 157.988 103.495) (end 161.788 103.495) (width 0.25) (layer B.Cu) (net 9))
 (segment (start 123.698 98.425) (end 123.698 103.505) (width 0.25) (layer B.Cu) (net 4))
 (segment (start 123.698 103.505) (end 128.778 103.505) (width 0.25) (layer B.Cu) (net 4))
 (via (at 174.498 116.205) (size 0.6) (drill 0.4) (layers F.Cu B.Cu) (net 4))
 (via (at 128.778 106.045) (size 0.6) (drill 0.4) (layers F.Cu B.Cu) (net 4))
 (segment (start 128.778 106.045) (end 128.778 103.505) (width 0.25) (layer B.Cu) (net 4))
 (segment (start 174.498 90.805) (end 174.498 93.345) (width 0.25) (layer B.Cu) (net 4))
 (segment (start 128.778 108.585) (end 128.778 106.045) (width 0.25) (layer F.Cu) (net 4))
 (segment (start 149.098 108.585) (end 128.778 108.585) (width 0.25) (layer F.Cu) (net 4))
 (segment (start 174.498 118.745) (end 151.638 118.745) (width 0.25) (layer F.Cu) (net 4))
 (segment (start 149.098 116.205) (end 149.098 108.585) (width 0.25) (layer F.Cu) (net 4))
 (segment (start 174.498 116.205) (end 174.498 118.745) (width 0.25) (layer F.Cu) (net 4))
 (segment (start 151.638 118.745) (end 151.638 116.205) (width 0.25) (layer F.Cu) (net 4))
 (segment (start 151.638 116.205) (end 149.098 116.205) (width 0.25) (layer F.Cu) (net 4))
 (segment (start 174.498 116.205) (end 174.498 113.665) (width 0.25) (layer B.Cu) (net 4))
 (segment (start 174.498 113.665) (end 177.038 113.665) (width 0.25) (layer B.Cu) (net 4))
 (via (at 177.038 113.665) (size 0.6) (drill 0.4) (layers F.Cu B.Cu) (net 4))
 (segment (start 177.038 113.665) (end 177.038 94.785) (width 0.25) (layer F.Cu) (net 4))
 (via (at 177.038 93.345) (size 0.6) (drill 0.4) (layers F.Cu B.Cu) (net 4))
 (segment (start 177.038 94.785) (end 177.038 93.345) (width 0.25) (layer F.Cu) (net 4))
 (via (at 177.038 93.345) (size 0.6) (drill 0.4) (layers F.Cu B.Cu) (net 4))
 (segment (start 177.038 93.345) (end 174.498 93.345) (width 0.25) (layer B.Cu) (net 4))
 (segment (start 128.778 98.425) (end 128.778 95.885) (width 0.25) (layer B.Cu) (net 11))
 (segment (start 174.498 111.125) (end 169.418 111.125) (width 0.25) (layer B.Cu) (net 13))
 (segment (start 169.418 108.585) (end 174.498 108.585) (width 0.25) (layer B.Cu) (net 14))
 (segment (start 169.418 103.505) (end 174.498 103.505) (width 0.25) (layer B.Cu) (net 16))
 (segment (start 174.498 106.045) (end 169.418 106.045) (width 0.25) (layer B.Cu) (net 15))
 (segment (start 136.061527 90.603473) (end 136.271 90.394) (width 0.25) (layer B.Cu) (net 2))
 (segment (start 135.509 90.805) (end 135.710527 90.603473) (width 0.25) (layer B.Cu) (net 2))
 (segment (start 121.698 95.925) (end 121.698 93.885) (width 0.25) (layer B.Cu) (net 2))
 (segment (start 133.858 90.805) (end 135.509 90.805) (width 0.25) (layer B.Cu) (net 2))
 (segment (start 121.698 93.885) (end 122.238 93.345) (width 0.25) (layer B.Cu) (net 2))
 (segment (start 122.238 93.345) (end 133.858 93.345) (width 0.25) (layer B.Cu) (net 2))
 (segment (start 135.710527 90.603473) (end 136.061527 90.603473) (width 0.25) (layer B.Cu) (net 2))
 (segment (start 133.858 93.345) (end 133.858 90.805) (width 0.25) (layer B.Cu) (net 2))
 (segment (start 136.398 101.092) (end 136.271 101.219) (width 0.25) (layer B.Cu) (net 3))
 (segment (start 126.198 95.925) (end 126.238 95.965) (width 0.25) (layer B.Cu) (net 3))
 (segment (start 126.238 95.965) (end 126.238 100.965) (width 0.25) (layer B.Cu) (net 3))
 (segment (start 123.698 95.925) (end 126.198 95.925) (width 0.25) (layer B.Cu) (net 3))
 (segment (start 126.238 100.965) (end 136.398 100.965) (width 0.25) (layer B.Cu) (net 3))
 (segment (start 136.398 100.965) (end 136.398 101.092) (width 0.25) (layer B.Cu) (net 3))
 (segment (start 146.304 98.679) (end 136.271 98.679) (width 0.25) (layer B.Cu) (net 17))
 (via (at 151.638 98.425) (size 0.6) (drill 0.4) (layers F.Cu B.Cu) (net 17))
 (segment (start 151.638 98.425) (end 146.304 98.679) (width 0.25) (layer B.Cu) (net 17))
 (segment (start 151.638 98.425) (end 151.638 113.665) (width 0.25) (layer F.Cu) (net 17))
 (via (at 151.638 113.665) (size 0.6) (drill 0.4) (layers F.Cu B.Cu) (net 17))
 (segment (start 156.718 113.665) (end 161.798 113.665) (width 0.25) (layer B.Cu) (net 17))
 (segment (start 151.638 113.665) (end 156.718 113.665) (width 0.25) (layer B.Cu) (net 17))
 (via (at 169.418 116.205) (size 0.6) (drill 0.4) (layers F.Cu B.Cu) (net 18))
 (segment (start 154.178 116.205) (end 169.418 116.205) (width 0.25) (layer F.Cu) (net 18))
 (via (at 154.178 88.265) (size 0.6) (drill 0.4) (layers F.Cu B.Cu) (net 18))
 (segment (start 154.178 88.265) (end 154.178 116.205) (width 0.25) (layer F.Cu) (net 18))
 (segment (start 161.798 88.265) (end 154.178 88.265) (width 0.25) (layer B.Cu) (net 18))
 (segment (start 169.418 113.665) (end 169.418 116.205) (width 0.25) (layer B.Cu) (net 18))
 (segment (start 149.098 93.345) (end 149.098 88.265) (width 0.25) (layer B.Cu) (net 18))
 (segment (start 136.398 93.345) (end 149.098 93.345) (width 0.25) (layer B.Cu) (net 18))
 (segment (start 149.098 88.265) (end 154.178 88.265) (width 0.25) (layer B.Cu) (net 18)))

